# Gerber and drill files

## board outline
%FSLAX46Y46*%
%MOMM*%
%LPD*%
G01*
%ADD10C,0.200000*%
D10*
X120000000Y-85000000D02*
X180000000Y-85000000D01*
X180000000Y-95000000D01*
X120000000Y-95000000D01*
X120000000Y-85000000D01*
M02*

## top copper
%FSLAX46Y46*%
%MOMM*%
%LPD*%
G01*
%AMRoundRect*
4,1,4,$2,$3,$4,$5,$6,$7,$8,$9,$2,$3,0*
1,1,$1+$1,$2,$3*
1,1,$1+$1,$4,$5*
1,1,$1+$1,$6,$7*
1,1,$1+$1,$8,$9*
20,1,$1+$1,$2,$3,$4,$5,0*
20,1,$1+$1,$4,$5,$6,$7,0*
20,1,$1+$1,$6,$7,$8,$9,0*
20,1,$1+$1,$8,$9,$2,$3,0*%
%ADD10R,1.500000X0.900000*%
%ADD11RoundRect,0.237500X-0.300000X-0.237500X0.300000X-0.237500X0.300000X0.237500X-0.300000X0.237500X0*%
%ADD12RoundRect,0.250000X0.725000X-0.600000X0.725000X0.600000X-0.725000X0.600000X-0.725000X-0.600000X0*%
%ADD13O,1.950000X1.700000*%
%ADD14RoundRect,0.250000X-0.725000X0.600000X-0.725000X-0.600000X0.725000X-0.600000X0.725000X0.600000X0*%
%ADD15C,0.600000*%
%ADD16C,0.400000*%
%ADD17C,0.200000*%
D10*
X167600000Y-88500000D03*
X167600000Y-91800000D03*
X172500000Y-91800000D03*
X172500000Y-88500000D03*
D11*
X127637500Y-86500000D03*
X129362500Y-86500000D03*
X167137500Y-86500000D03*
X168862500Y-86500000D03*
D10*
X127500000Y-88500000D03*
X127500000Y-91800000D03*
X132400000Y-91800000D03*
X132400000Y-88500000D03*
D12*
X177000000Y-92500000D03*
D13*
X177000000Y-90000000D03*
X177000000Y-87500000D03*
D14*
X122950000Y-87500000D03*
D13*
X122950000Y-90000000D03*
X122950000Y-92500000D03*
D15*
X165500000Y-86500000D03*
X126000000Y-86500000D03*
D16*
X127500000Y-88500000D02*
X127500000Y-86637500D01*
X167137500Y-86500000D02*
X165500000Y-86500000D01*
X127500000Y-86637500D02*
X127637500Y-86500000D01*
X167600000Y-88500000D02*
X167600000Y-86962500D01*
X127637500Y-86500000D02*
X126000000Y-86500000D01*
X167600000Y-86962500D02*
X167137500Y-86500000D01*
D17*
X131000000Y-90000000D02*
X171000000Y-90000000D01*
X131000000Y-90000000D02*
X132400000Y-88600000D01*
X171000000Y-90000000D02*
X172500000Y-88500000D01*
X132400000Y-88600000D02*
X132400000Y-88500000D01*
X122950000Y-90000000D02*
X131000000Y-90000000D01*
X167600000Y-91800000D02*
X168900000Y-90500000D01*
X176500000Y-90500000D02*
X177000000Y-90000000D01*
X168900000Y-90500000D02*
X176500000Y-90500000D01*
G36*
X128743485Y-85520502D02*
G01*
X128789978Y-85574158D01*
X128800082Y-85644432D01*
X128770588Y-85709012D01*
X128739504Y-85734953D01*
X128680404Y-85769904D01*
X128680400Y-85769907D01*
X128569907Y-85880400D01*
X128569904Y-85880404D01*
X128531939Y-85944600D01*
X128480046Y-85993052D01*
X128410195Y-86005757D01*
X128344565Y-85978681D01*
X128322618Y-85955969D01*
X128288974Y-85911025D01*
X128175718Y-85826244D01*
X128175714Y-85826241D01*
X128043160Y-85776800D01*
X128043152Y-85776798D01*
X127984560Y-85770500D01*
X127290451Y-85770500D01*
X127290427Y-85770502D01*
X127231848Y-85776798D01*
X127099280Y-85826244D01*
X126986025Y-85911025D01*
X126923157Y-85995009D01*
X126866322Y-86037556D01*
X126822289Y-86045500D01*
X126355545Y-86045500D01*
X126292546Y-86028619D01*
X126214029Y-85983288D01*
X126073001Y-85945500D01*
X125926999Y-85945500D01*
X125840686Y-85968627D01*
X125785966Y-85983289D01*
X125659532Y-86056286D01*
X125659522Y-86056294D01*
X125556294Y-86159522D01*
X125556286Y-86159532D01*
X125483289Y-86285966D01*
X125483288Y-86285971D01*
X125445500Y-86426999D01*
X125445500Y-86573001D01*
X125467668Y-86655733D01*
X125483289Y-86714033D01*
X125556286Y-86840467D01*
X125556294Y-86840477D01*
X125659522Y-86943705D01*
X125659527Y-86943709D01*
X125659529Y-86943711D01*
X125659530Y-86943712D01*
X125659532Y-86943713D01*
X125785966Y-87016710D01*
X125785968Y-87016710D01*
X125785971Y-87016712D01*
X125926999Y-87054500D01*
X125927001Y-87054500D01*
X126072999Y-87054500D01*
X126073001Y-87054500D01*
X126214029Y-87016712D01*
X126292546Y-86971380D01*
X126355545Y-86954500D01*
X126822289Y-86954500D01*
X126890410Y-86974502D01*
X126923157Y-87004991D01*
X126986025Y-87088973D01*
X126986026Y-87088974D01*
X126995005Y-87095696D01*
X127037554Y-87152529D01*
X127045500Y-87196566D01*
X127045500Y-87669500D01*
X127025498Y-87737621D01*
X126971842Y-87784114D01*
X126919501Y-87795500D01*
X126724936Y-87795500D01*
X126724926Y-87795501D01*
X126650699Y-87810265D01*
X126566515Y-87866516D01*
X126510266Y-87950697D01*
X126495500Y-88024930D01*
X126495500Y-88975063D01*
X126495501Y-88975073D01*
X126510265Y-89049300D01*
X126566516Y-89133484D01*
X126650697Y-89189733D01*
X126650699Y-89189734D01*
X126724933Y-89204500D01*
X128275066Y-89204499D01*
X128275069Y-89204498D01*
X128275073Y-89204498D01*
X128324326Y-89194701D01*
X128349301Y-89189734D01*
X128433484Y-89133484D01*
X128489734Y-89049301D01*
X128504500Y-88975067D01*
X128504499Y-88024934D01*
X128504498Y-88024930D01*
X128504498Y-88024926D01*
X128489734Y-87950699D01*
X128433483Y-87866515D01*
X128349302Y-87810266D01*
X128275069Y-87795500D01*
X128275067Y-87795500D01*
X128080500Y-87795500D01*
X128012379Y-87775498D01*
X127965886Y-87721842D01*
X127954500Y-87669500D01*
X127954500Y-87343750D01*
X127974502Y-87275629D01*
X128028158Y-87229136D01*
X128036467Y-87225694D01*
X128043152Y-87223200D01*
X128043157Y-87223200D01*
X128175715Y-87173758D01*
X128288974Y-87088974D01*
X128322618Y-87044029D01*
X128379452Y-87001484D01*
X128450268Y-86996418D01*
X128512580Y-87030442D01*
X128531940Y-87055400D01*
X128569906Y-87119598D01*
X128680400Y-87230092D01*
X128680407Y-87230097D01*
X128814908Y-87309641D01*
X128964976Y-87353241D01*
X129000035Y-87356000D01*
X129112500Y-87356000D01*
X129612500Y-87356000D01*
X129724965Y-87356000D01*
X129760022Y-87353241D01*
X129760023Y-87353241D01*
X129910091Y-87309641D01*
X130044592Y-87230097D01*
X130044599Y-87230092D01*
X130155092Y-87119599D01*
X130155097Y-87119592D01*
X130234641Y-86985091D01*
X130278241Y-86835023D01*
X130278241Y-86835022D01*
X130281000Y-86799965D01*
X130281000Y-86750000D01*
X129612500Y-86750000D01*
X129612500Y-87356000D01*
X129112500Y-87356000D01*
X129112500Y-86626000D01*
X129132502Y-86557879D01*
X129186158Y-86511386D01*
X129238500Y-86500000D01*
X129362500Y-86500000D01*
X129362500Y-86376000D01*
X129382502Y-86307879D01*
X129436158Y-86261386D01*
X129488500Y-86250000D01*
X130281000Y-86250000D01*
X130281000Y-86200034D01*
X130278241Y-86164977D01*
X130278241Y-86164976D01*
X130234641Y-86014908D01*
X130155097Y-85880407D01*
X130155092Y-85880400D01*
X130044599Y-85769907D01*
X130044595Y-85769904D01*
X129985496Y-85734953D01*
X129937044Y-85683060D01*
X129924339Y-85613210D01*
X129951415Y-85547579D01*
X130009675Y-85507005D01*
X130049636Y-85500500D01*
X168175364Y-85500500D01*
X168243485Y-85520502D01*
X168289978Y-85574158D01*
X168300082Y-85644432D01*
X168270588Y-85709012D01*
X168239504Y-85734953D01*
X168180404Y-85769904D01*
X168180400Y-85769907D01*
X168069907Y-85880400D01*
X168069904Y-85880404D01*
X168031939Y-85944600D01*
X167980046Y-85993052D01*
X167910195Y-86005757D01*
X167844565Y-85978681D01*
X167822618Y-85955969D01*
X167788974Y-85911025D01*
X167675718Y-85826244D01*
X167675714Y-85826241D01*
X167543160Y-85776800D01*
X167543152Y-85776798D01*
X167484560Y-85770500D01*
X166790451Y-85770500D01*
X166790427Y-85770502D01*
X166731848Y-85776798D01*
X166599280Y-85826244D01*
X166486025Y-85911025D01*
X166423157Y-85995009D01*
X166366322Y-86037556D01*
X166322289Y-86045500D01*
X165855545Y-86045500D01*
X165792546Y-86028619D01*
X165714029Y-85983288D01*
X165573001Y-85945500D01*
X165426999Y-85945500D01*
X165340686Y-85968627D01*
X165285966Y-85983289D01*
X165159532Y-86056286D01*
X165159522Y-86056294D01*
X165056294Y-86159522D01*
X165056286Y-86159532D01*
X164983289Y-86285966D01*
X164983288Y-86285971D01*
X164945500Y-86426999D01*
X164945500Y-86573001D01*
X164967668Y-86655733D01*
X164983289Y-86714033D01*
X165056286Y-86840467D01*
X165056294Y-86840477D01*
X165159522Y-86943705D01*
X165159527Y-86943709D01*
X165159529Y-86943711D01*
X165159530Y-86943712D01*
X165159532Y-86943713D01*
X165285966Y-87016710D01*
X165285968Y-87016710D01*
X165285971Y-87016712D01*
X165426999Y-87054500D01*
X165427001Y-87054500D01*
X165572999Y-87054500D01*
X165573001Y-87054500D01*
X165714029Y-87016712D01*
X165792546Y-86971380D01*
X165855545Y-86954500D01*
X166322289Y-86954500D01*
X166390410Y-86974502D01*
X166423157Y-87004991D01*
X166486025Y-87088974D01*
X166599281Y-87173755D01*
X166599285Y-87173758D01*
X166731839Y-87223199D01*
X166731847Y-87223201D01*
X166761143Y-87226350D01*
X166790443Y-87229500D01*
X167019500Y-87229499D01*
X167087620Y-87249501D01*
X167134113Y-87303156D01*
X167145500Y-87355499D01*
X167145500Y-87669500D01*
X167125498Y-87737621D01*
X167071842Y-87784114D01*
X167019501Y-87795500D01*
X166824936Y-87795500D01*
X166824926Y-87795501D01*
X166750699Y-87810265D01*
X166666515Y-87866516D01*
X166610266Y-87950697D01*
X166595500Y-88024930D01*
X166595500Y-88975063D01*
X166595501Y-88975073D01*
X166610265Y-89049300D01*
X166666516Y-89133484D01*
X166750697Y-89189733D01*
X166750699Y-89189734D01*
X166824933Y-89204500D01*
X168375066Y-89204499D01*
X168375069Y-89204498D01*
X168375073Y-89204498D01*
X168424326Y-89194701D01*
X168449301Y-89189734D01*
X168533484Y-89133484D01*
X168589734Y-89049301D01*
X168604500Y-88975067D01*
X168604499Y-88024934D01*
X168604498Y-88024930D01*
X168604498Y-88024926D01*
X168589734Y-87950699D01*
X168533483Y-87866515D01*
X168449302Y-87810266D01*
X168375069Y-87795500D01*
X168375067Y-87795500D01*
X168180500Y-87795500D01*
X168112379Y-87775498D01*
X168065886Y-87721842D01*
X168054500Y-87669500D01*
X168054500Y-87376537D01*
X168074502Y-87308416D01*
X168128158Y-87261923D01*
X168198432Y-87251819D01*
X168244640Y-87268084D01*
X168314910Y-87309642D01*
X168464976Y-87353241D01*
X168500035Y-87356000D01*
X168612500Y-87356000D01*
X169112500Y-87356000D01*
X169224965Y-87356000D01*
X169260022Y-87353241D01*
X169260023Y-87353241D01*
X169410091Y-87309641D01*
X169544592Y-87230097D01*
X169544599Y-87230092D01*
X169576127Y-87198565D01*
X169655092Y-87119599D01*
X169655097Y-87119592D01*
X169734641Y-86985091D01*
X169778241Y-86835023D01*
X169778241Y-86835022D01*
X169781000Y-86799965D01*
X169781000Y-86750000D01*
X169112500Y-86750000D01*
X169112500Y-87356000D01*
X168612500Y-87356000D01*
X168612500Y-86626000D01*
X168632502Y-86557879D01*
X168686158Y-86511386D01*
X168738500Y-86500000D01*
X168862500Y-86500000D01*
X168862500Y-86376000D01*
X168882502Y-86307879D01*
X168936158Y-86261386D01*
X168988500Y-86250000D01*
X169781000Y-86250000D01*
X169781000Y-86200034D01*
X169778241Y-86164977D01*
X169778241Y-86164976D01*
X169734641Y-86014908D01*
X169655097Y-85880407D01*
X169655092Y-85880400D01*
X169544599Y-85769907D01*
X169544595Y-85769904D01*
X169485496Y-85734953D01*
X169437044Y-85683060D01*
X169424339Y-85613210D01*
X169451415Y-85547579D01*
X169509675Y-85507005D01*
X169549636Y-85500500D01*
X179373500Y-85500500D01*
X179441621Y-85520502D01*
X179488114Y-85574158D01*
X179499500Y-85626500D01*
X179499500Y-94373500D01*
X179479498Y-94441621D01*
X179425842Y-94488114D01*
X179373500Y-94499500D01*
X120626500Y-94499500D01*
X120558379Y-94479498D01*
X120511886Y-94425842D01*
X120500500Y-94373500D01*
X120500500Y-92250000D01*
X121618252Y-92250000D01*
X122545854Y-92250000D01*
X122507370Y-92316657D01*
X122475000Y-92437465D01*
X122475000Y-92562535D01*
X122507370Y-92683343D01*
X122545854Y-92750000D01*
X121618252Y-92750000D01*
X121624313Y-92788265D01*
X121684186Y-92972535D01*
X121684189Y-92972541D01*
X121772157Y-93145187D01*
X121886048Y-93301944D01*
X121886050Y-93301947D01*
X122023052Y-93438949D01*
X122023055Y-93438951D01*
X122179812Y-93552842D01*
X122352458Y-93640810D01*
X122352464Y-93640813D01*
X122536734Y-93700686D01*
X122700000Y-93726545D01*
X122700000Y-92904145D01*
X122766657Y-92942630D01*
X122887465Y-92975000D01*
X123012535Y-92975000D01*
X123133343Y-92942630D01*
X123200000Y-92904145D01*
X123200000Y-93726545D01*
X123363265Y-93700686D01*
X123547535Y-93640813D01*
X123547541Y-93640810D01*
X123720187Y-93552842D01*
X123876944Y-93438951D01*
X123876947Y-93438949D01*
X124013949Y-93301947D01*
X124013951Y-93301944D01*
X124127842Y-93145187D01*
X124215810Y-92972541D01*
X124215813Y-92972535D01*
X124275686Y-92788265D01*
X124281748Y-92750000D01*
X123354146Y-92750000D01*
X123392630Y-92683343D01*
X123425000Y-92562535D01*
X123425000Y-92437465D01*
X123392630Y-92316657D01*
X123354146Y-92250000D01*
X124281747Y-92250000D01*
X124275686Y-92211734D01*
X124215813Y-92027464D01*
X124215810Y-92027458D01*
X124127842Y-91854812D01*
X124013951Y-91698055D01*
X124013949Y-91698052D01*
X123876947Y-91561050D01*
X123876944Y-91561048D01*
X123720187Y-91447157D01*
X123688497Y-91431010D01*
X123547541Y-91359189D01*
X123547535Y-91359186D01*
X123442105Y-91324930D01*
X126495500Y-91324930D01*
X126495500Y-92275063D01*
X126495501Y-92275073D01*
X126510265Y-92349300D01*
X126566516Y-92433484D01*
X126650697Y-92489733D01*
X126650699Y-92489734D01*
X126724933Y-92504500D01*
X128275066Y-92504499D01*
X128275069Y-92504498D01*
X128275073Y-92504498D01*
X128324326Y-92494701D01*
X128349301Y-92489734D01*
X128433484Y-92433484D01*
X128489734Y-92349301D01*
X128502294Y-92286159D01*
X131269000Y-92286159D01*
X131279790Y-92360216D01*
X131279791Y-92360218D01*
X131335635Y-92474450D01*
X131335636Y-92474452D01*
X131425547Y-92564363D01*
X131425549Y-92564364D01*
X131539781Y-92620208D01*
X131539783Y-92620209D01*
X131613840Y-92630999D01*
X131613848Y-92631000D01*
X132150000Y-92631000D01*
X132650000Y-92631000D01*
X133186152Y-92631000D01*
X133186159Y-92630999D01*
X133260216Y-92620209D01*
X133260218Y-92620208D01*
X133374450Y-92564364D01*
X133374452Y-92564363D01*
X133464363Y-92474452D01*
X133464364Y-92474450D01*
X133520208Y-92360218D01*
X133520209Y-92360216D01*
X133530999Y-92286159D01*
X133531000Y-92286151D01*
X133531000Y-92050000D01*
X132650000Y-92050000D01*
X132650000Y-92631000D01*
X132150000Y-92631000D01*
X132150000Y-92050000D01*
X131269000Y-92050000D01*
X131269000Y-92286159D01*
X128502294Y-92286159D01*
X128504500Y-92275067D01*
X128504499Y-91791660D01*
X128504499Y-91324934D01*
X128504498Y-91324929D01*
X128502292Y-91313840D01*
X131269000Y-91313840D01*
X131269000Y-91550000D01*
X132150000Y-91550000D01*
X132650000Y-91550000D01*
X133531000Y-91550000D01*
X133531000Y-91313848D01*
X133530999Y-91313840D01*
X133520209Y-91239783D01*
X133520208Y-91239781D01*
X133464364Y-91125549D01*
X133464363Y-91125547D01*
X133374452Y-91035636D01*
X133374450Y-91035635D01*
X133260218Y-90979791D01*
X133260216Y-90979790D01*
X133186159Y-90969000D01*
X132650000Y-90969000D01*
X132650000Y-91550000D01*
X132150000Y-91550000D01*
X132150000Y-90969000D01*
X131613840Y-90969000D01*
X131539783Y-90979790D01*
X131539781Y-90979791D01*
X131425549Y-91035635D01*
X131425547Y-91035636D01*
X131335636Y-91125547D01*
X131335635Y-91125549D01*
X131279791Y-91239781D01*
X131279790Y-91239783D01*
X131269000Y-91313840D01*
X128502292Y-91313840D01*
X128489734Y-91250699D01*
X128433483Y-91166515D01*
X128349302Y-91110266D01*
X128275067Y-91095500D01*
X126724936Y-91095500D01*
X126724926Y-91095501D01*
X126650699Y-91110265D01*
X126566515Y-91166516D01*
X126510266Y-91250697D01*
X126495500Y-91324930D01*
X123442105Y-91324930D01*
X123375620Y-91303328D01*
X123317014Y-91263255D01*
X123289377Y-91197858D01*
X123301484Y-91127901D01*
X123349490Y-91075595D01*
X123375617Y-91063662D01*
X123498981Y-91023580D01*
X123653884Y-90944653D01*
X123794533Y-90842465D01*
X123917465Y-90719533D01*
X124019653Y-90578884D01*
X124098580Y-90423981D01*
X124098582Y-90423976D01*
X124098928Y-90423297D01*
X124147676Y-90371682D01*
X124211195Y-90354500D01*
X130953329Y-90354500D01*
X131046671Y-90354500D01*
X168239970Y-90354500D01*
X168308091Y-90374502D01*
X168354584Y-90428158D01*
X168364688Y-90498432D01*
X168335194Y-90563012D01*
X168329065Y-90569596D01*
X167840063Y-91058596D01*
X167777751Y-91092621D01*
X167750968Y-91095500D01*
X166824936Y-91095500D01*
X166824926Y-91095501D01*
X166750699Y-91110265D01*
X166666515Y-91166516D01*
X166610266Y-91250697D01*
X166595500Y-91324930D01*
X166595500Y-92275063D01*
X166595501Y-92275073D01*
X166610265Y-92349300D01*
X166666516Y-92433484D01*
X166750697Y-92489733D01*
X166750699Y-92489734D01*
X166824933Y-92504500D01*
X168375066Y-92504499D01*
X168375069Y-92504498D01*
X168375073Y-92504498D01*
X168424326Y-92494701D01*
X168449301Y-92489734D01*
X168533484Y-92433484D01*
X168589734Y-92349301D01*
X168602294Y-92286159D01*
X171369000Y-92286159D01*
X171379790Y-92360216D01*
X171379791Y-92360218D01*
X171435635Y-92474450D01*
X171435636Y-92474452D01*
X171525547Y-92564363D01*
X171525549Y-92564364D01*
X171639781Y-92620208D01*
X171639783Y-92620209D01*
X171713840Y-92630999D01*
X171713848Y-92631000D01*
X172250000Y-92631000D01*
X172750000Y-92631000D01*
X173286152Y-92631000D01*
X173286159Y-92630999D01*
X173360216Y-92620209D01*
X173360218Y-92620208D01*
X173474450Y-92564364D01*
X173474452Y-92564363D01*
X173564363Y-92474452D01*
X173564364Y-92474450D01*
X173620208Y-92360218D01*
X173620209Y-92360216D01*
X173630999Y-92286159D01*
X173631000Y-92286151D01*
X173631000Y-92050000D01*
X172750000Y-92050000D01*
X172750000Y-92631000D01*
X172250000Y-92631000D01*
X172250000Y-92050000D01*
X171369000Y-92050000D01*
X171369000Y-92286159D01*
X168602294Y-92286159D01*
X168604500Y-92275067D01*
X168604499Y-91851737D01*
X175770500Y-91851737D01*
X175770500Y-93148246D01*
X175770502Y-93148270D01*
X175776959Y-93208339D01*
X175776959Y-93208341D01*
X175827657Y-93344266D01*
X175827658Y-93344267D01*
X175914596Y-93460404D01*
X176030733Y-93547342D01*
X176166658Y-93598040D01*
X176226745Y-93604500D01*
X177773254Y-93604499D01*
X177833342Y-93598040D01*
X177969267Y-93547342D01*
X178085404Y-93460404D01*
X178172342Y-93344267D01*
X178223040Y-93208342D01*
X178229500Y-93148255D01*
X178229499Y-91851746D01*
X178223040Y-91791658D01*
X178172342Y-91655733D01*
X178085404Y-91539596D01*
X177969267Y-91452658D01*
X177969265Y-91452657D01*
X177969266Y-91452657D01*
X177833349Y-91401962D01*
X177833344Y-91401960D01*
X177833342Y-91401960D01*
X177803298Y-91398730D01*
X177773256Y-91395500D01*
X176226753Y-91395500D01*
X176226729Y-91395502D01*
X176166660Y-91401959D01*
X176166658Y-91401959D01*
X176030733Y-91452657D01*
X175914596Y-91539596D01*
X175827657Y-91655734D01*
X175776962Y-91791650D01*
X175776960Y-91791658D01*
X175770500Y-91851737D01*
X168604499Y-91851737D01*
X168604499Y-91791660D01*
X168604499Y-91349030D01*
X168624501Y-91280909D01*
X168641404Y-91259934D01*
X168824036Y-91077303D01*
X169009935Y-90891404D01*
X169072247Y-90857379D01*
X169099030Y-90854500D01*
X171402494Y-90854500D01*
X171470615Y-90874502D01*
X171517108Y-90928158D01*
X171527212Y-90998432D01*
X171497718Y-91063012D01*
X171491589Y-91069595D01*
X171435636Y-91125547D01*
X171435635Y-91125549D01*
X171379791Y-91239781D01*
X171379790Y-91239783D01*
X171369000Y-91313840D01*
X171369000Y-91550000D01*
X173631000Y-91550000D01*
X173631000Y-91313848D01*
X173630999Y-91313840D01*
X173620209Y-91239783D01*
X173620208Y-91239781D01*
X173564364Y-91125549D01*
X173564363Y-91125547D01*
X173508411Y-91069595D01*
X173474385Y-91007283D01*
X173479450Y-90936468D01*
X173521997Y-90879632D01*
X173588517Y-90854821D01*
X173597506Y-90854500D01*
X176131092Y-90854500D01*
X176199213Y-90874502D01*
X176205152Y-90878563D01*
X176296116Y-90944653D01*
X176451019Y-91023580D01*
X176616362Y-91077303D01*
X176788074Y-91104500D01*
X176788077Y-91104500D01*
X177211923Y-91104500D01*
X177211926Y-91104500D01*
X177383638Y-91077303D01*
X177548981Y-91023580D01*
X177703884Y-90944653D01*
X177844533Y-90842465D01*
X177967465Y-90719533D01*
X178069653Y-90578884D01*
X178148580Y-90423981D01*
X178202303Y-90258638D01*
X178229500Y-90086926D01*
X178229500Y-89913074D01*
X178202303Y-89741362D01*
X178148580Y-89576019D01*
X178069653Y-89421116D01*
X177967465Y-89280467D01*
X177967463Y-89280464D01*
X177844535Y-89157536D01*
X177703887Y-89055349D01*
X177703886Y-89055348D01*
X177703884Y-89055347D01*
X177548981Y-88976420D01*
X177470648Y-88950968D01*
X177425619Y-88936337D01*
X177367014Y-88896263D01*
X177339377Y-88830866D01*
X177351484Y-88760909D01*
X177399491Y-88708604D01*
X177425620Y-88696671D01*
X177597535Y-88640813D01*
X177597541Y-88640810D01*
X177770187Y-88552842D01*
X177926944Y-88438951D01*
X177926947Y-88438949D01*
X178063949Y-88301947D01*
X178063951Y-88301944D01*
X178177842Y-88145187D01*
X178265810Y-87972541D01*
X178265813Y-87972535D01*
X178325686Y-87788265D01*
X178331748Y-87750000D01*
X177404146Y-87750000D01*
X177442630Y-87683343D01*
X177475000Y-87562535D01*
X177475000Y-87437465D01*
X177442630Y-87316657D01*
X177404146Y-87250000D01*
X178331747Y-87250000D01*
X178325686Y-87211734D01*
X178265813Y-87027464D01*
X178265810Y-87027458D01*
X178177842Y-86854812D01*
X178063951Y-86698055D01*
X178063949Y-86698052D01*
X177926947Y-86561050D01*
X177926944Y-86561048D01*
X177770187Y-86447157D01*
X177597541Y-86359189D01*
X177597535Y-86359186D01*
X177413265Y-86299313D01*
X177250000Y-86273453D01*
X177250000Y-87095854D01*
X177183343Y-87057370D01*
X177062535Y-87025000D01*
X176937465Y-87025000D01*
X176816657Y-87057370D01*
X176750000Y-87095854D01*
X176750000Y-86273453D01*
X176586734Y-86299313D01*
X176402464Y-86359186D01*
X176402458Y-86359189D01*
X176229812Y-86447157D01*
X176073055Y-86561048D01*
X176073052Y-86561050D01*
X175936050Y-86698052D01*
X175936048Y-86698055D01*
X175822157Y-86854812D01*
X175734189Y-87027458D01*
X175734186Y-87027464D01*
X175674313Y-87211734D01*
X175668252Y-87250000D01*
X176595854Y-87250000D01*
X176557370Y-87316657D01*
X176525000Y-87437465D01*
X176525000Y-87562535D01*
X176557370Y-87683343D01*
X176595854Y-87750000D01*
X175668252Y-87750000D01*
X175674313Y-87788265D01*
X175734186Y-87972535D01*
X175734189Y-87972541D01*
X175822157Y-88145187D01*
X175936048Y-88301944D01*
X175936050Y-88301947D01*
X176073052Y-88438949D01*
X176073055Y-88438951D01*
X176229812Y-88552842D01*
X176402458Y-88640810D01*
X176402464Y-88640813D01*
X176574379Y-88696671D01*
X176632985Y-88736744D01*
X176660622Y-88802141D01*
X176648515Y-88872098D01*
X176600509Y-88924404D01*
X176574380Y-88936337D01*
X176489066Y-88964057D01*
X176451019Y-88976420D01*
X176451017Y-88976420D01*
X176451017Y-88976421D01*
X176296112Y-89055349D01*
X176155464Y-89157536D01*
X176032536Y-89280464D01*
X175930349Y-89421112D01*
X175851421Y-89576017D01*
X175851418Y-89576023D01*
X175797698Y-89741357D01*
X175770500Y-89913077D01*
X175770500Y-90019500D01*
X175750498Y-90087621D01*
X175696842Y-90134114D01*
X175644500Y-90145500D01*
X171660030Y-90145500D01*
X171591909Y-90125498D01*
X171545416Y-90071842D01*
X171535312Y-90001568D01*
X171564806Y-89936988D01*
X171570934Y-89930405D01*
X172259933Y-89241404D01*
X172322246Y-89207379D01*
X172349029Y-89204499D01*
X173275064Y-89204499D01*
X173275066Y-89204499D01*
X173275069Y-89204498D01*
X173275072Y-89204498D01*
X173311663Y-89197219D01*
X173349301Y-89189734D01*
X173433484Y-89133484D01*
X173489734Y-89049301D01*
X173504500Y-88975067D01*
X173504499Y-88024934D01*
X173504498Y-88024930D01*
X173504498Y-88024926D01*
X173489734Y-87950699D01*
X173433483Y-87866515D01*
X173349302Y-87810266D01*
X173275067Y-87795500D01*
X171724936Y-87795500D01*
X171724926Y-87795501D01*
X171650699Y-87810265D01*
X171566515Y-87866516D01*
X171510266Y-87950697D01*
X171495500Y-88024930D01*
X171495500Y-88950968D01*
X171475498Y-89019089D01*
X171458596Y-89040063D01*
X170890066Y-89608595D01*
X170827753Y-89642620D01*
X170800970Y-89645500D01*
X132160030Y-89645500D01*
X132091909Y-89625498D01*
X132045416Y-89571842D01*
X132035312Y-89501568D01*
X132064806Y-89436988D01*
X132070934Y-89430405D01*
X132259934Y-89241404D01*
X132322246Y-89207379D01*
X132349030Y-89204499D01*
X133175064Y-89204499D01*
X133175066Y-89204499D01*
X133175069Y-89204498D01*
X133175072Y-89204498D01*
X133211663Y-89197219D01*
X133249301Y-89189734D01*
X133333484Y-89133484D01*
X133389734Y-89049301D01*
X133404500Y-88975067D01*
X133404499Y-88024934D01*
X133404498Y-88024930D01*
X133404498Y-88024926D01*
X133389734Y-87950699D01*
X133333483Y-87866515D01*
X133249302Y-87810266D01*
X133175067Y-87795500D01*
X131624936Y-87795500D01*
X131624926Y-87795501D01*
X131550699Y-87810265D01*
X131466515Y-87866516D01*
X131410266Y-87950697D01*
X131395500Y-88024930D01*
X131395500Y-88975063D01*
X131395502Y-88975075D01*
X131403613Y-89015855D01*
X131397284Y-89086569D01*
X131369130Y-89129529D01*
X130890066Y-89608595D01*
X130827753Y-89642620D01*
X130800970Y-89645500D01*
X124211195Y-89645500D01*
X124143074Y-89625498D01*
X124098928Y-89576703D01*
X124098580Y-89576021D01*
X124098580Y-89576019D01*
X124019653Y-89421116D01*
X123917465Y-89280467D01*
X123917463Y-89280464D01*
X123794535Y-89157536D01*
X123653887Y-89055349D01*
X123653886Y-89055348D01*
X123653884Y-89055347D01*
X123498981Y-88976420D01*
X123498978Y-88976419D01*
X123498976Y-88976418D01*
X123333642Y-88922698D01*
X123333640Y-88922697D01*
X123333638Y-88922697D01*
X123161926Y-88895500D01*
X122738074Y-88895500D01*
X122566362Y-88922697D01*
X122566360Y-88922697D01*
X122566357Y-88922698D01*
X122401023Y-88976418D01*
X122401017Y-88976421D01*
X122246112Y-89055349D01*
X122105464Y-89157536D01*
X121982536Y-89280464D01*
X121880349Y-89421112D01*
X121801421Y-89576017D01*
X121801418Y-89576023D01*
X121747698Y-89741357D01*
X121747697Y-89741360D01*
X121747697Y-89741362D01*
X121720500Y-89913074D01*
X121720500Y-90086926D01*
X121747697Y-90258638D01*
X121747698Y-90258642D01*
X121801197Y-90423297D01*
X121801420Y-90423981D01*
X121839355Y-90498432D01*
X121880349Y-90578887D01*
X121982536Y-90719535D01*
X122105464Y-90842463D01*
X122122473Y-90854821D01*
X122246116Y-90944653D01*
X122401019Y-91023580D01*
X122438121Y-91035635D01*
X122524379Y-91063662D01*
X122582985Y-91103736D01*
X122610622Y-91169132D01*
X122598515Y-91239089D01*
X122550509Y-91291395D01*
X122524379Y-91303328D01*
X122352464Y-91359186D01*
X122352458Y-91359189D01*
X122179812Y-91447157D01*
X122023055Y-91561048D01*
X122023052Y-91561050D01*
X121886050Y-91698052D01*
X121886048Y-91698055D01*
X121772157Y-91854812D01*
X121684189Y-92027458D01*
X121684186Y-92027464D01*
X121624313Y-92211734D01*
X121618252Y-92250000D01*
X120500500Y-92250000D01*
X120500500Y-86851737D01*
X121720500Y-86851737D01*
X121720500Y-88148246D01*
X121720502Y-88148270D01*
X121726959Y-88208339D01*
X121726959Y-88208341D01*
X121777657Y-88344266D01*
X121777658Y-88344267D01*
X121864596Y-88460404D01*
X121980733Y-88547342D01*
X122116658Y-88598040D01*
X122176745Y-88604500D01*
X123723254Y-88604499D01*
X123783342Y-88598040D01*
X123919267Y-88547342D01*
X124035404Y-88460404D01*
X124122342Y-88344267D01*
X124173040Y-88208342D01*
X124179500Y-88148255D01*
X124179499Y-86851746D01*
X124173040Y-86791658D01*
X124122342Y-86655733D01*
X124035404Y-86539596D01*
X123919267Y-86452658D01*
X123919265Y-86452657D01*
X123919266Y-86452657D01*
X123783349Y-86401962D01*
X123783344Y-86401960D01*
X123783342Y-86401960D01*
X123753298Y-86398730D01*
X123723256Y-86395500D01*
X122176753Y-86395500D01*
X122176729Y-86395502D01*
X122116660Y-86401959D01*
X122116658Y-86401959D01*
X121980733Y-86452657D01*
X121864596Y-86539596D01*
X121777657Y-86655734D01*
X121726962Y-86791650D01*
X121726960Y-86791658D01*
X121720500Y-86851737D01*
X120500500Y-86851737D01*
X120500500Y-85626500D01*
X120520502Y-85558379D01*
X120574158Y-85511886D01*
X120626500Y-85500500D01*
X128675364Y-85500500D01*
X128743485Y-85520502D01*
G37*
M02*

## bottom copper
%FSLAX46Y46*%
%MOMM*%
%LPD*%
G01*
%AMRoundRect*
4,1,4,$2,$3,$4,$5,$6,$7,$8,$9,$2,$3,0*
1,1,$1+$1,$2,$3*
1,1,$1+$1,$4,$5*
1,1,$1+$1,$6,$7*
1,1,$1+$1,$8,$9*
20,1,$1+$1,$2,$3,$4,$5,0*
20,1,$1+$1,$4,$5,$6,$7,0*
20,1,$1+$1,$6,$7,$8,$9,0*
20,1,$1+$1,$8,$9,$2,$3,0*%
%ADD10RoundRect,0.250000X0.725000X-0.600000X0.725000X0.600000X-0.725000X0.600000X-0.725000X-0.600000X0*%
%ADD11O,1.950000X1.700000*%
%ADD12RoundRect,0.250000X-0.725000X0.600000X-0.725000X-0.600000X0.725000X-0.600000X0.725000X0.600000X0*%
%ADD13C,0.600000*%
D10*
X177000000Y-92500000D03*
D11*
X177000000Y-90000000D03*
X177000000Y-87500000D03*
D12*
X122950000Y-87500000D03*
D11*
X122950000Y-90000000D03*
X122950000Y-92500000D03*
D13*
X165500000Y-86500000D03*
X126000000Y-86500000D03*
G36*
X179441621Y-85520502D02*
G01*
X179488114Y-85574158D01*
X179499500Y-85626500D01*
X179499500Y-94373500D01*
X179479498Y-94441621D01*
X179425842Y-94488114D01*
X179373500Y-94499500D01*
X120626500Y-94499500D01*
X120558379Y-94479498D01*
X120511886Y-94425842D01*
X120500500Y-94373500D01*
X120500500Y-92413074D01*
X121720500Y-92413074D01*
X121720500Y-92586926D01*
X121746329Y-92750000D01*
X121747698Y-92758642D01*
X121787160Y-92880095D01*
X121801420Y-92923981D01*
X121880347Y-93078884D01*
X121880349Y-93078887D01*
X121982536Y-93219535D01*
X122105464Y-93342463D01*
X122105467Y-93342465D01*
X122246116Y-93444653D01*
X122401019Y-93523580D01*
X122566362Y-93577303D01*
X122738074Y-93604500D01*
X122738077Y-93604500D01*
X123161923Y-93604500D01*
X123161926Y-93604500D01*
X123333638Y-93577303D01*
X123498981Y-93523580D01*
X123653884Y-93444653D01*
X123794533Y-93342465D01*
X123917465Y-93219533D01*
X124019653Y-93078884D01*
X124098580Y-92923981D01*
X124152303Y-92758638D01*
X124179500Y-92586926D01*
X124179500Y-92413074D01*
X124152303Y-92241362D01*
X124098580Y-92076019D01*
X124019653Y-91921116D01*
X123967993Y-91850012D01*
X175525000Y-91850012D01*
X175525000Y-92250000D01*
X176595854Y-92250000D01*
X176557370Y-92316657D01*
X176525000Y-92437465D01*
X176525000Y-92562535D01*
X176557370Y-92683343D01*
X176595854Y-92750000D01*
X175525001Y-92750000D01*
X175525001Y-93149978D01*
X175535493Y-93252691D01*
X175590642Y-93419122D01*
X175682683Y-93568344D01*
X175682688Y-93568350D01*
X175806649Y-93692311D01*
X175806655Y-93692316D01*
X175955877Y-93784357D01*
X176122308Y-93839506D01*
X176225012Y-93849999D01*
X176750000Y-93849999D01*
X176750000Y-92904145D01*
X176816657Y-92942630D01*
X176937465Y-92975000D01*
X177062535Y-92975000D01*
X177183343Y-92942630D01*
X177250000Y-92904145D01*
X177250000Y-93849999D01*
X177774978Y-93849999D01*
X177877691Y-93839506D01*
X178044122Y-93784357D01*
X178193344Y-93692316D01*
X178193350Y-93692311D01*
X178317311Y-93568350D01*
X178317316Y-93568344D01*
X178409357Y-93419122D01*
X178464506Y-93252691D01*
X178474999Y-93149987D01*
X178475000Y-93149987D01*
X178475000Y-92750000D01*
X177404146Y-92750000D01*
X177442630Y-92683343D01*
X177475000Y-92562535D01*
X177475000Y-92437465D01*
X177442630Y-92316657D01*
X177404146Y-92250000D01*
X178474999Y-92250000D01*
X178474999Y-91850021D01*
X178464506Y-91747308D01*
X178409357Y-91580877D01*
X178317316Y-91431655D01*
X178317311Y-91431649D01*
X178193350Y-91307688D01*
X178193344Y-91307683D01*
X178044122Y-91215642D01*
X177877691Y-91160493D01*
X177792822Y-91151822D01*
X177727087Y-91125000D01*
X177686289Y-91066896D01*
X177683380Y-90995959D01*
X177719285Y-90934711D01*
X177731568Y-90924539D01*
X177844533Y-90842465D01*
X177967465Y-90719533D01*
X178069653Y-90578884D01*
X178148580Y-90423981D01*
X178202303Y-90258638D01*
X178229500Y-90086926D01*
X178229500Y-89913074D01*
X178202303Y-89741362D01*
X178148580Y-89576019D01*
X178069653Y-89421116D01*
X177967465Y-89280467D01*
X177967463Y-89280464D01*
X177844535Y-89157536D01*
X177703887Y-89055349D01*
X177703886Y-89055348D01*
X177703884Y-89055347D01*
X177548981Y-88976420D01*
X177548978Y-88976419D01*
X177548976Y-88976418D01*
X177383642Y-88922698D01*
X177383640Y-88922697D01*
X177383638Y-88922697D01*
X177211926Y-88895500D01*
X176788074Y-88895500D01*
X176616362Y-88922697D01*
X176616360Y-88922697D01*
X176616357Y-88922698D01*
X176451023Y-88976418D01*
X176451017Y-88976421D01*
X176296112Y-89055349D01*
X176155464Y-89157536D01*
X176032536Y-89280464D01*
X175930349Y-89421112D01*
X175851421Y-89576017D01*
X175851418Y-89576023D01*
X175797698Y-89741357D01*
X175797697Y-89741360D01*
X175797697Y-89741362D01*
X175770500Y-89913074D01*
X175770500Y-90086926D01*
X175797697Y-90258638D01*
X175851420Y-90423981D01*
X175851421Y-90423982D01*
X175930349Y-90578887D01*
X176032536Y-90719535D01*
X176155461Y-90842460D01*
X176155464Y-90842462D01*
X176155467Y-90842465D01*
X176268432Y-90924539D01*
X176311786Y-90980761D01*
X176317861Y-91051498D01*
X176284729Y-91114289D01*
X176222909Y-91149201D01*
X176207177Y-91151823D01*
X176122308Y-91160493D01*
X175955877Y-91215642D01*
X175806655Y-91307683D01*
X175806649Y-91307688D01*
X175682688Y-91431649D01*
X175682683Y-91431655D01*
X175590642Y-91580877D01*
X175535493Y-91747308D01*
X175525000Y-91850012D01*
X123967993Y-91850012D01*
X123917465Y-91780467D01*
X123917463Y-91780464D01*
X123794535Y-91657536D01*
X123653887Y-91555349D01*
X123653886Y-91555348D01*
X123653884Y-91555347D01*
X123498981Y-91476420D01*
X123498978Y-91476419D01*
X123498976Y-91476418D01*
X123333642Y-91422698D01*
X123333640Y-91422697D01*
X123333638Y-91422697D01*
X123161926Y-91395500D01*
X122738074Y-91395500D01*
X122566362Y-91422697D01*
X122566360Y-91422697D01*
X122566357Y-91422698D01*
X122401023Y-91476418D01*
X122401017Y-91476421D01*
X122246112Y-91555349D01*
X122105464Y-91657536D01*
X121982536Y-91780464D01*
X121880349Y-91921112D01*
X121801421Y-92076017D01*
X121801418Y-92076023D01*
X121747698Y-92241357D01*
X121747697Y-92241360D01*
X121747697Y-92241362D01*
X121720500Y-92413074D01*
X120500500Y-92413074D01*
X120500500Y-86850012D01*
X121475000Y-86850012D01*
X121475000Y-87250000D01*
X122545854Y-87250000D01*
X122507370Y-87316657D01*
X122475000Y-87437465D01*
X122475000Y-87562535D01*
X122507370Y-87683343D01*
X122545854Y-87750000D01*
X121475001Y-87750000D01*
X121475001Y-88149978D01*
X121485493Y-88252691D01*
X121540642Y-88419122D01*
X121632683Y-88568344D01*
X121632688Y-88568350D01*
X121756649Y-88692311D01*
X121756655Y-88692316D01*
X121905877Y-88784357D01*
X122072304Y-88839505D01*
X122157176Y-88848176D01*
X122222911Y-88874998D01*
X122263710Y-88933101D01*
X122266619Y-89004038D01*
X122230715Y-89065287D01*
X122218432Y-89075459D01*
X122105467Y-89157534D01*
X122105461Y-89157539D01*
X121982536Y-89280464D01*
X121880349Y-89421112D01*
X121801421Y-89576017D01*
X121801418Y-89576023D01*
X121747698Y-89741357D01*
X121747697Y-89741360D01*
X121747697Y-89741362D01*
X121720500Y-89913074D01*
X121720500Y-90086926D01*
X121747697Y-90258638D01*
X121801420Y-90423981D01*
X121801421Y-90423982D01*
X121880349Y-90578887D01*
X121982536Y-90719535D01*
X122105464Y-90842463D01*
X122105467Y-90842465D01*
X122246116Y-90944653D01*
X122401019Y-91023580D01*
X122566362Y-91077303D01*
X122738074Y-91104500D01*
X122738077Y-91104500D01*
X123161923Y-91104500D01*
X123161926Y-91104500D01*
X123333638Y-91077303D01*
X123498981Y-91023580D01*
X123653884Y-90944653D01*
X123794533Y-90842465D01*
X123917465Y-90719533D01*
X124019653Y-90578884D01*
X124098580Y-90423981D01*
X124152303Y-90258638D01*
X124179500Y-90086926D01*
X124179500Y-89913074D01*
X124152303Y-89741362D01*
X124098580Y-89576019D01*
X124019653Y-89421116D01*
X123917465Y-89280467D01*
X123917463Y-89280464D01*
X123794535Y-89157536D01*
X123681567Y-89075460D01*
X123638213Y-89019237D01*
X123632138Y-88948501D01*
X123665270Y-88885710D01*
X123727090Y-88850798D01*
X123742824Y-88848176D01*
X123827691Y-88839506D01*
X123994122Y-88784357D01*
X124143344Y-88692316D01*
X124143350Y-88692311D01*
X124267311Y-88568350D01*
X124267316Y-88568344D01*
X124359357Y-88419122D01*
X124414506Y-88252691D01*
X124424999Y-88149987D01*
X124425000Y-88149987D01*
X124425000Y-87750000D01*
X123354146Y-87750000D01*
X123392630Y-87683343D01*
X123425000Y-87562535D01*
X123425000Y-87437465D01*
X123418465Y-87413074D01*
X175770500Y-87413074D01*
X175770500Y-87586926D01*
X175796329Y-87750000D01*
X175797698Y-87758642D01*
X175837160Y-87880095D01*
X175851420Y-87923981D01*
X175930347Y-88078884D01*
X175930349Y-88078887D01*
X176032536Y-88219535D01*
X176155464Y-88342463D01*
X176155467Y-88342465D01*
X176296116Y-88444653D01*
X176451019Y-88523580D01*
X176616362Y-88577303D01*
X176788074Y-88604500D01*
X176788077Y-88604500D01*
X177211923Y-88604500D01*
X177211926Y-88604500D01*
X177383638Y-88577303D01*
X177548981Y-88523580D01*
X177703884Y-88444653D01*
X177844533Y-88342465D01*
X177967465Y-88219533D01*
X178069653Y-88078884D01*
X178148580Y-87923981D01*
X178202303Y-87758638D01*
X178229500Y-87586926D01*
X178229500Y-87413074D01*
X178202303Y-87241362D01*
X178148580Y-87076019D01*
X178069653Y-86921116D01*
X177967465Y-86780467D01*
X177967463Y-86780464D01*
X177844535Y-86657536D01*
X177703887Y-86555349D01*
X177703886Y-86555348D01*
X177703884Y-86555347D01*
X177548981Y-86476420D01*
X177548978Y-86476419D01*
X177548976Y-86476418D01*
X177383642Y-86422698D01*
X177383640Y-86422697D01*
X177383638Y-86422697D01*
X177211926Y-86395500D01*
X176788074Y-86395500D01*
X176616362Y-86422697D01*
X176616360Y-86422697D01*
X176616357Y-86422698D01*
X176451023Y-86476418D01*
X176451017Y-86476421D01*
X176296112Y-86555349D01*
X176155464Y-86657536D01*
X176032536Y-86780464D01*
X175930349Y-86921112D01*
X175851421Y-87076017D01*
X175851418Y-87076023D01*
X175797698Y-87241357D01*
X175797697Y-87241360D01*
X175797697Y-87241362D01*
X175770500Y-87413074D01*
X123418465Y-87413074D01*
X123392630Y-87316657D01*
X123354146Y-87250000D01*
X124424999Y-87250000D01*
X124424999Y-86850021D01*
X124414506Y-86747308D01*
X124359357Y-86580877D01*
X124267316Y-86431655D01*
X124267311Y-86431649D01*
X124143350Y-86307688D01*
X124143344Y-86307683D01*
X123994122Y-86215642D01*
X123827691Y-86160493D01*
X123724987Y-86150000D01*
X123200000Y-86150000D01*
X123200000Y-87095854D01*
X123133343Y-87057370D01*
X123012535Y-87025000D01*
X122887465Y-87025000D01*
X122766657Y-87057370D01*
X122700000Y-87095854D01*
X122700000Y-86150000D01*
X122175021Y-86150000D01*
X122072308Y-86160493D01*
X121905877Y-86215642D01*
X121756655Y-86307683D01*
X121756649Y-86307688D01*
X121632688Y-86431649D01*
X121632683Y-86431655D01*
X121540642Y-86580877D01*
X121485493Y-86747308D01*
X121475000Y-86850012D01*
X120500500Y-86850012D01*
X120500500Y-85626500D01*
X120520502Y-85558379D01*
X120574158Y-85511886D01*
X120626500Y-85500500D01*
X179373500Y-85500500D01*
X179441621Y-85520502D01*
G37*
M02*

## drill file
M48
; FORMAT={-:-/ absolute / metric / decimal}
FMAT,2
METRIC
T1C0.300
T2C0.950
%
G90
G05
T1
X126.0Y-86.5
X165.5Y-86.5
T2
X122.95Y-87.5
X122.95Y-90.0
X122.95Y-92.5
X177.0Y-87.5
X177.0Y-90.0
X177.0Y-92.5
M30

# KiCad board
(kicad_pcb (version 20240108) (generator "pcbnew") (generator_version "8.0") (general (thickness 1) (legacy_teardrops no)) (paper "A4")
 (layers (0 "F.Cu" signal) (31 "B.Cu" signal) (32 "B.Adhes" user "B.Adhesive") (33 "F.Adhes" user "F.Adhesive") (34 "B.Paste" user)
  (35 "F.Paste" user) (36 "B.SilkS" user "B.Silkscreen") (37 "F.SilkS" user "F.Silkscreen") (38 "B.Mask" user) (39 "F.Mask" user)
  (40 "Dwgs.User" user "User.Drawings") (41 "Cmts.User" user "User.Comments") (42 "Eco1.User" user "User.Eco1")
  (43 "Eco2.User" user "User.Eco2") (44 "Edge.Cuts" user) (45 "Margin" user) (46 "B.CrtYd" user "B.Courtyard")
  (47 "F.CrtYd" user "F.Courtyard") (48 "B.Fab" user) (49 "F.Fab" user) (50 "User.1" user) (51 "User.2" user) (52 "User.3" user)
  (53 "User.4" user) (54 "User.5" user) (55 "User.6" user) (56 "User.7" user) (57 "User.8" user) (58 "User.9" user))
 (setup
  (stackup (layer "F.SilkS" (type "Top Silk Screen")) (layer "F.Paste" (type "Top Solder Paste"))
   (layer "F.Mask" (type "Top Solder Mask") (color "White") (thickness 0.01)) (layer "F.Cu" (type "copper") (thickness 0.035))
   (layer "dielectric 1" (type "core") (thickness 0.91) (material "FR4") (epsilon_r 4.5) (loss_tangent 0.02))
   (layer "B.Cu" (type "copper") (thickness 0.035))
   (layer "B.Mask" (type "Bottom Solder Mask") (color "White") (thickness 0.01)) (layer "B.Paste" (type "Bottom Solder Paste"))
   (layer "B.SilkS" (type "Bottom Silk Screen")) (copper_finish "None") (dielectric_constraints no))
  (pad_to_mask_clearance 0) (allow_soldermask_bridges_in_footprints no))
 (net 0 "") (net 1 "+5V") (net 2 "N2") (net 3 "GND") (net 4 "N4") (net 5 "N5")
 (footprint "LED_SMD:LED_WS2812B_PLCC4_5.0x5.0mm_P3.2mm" (layer "F.Cu") (at 170.05 90.15)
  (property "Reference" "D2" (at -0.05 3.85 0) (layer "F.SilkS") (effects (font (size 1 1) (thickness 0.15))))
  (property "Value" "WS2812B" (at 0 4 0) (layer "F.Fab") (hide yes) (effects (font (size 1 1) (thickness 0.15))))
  (pad "1" smd rect (at -2.45 -1.65) (size 1.5 0.9) (layers "F.Cu" "F.Paste" "F.Mask") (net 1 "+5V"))
  (pad "2" smd rect (at -2.45 1.65) (size 1.5 0.9) (layers "F.Cu" "F.Paste" "F.Mask") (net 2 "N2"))
  (pad "3" smd rect (at 2.45 1.65) (size 1.5 0.9) (layers "F.Cu" "F.Paste" "F.Mask") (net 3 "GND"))
  (pad "4" smd rect (at 2.45 -1.65) (size 1.5 0.9) (layers "F.Cu" "F.Paste" "F.Mask") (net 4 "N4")))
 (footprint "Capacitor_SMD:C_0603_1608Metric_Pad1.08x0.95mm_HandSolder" (layer "F.Cu") (at 128.5 86.5)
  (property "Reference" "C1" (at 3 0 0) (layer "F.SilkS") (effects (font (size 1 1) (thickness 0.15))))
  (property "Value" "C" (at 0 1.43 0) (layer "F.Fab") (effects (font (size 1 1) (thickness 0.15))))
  (pad "1" smd roundrect (at -0.8625 0) (size 1.075 0.95) (layers "F.Cu" "F.Paste" "F.Mask") (roundrect_rratio 0.25) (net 1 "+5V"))
  (pad "2" smd roundrect (at 0.8625 0) (size 1.075 0.95) (layers "F.Cu" "F.Paste" "F.Mask") (roundrect_rratio 0.25) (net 3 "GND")))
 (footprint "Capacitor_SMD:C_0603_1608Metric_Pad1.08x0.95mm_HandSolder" (layer "F.Cu") (at 168 86.5)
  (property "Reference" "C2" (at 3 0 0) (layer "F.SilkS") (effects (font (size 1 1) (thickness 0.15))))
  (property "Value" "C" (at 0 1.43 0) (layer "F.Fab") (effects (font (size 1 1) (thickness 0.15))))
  (pad "1" smd roundrect (at -0.8625 0) (size 1.075 0.95) (layers "F.Cu" "F.Paste" "F.Mask") (roundrect_rratio 0.25) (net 1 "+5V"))
  (pad "2" smd roundrect (at 0.8625 0) (size 1.075 0.95) (layers "F.Cu" "F.Paste" "F.Mask") (roundrect_rratio 0.25) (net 3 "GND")))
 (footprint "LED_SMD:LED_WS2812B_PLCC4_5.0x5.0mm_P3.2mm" (layer "F.Cu") (at 129.95 90.15)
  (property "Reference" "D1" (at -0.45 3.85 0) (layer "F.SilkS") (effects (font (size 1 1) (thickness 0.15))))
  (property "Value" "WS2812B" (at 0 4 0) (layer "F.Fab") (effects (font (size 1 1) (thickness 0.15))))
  (pad "1" smd rect (at -2.45 -1.65) (size 1.5 0.9) (layers "F.Cu" "F.Paste" "F.Mask") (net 1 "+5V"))
  (pad "2" smd rect (at -2.45 1.65) (size 1.5 0.9) (layers "F.Cu" "F.Paste" "F.Mask") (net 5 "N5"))
  (pad "3" smd rect (at 2.45 1.65) (size 1.5 0.9) (layers "F.Cu" "F.Paste" "F.Mask") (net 3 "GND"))
  (pad "4" smd rect (at 2.45 -1.65) (size 1.5 0.9) (layers "F.Cu" "F.Paste" "F.Mask") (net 4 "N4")))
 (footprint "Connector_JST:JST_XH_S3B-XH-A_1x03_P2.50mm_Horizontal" (layer "F.Cu") (at 177 92.5 90)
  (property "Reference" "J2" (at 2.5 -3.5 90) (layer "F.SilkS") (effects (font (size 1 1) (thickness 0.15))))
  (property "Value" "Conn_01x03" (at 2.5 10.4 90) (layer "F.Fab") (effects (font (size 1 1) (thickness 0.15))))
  (pad "1" thru_hole roundrect (at 0 0 90) (size 1.7 1.95) (drill 0.95) (layers "*.Cu" "*.Mask") (remove_unused_layers no)
   (roundrect_rratio 0.147059) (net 1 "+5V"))
  (pad "2" thru_hole oval (at 2.5 0 90) (size 1.7 1.95) (drill 0.95) (layers "*.Cu" "*.Mask") (remove_unused_layers no) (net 2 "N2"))
  (pad "3" thru_hole oval (at 5 0 90) (size 1.7 1.95) (drill 0.95) (layers "*.Cu" "*.Mask") (remove_unused_layers no) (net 3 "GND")))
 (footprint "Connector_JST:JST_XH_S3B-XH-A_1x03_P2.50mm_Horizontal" (layer "F.Cu") (at 122.95 87.5 -90)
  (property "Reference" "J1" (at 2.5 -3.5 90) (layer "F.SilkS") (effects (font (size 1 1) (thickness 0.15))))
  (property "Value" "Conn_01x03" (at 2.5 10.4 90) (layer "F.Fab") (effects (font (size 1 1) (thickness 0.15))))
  (pad "1" thru_hole roundrect (at 0 0 270) (size 1.7 1.95) (drill 0.95) (layers "*.Cu" "*.Mask") (remove_unused_layers no)
   (roundrect_rratio 0.147059) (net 1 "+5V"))
  (pad "2" thru_hole oval (at 2.5 0 270) (size 1.7 1.95) (drill 0.95) (layers "*.Cu" "*.Mask") (remove_unused_layers no) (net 4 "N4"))
  (pad "3" thru_hole oval (at 5 0 270) (size 1.7 1.95) (drill 0.95) (layers "*.Cu" "*.Mask") (remove_unused_layers no) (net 3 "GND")))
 (gr_rect (start 120 85) (end 180 95) (stroke (width 0.2) (type default)) (fill none) (layer "Edge.Cuts"))
 (segment (start 127.5 88.5) (end 127.5 86.6375) (width 0.4) (layer "F.Cu") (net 1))
 (segment (start 167.1375 86.5) (end 165.5 86.5) (width 0.4) (layer "F.Cu") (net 1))
 (segment (start 127.5 86.6375) (end 127.6375 86.5) (width 0.4) (layer "F.Cu") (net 1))
 (segment (start 167.6 88.5) (end 167.6 86.9625) (width 0.4) (layer "F.Cu") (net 1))
 (segment (start 127.6375 86.5) (end 126 86.5) (width 0.4) (layer "F.Cu") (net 1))
 (segment (start 167.6 86.9625) (end 167.1375 86.5) (width 0.4) (layer "F.Cu") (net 1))
 (via (at 165.5 86.5) (size 0.6) (drill 0.3) (layers "F.Cu" "B.Cu") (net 1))
 (via (at 126 86.5) (size 0.6) (drill 0.3) (layers "F.Cu" "B.Cu") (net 1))
 (segment (start 131 90) (end 171 90) (width 0.2) (layer "F.Cu") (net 4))
 (segment (start 131 90) (end 132.4 88.6) (width 0.2) (layer "F.Cu") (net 4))
 (segment (start 171 90) (end 172.5 88.5) (width 0.2) (layer "F.Cu") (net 4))
 (segment (start 132.4 88.6) (end 132.4 88.5) (width 0.2) (layer "F.Cu") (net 4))
 (segment (start 122.95 90) (end 131 90) (width 0.2) (layer "F.Cu") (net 4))
 (segment (start 167.6 91.8) (end 168.9 90.5) (width 0.2) (layer "F.Cu") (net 2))
 (segment (start 176.5 90.5) (end 177 90) (width 0.2) (layer "F.Cu") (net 2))
 (segment (start 168.9 90.5) (end 176.5 90.5) (width 0.2) (layer "F.Cu") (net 2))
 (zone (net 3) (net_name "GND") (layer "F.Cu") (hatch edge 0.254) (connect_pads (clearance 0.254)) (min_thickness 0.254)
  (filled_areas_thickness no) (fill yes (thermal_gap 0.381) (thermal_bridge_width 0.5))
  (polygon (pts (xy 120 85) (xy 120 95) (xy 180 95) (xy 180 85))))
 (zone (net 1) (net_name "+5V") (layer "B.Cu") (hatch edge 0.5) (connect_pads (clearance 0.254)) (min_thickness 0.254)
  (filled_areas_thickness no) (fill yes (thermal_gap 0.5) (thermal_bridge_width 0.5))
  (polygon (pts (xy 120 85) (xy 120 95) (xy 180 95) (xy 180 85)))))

